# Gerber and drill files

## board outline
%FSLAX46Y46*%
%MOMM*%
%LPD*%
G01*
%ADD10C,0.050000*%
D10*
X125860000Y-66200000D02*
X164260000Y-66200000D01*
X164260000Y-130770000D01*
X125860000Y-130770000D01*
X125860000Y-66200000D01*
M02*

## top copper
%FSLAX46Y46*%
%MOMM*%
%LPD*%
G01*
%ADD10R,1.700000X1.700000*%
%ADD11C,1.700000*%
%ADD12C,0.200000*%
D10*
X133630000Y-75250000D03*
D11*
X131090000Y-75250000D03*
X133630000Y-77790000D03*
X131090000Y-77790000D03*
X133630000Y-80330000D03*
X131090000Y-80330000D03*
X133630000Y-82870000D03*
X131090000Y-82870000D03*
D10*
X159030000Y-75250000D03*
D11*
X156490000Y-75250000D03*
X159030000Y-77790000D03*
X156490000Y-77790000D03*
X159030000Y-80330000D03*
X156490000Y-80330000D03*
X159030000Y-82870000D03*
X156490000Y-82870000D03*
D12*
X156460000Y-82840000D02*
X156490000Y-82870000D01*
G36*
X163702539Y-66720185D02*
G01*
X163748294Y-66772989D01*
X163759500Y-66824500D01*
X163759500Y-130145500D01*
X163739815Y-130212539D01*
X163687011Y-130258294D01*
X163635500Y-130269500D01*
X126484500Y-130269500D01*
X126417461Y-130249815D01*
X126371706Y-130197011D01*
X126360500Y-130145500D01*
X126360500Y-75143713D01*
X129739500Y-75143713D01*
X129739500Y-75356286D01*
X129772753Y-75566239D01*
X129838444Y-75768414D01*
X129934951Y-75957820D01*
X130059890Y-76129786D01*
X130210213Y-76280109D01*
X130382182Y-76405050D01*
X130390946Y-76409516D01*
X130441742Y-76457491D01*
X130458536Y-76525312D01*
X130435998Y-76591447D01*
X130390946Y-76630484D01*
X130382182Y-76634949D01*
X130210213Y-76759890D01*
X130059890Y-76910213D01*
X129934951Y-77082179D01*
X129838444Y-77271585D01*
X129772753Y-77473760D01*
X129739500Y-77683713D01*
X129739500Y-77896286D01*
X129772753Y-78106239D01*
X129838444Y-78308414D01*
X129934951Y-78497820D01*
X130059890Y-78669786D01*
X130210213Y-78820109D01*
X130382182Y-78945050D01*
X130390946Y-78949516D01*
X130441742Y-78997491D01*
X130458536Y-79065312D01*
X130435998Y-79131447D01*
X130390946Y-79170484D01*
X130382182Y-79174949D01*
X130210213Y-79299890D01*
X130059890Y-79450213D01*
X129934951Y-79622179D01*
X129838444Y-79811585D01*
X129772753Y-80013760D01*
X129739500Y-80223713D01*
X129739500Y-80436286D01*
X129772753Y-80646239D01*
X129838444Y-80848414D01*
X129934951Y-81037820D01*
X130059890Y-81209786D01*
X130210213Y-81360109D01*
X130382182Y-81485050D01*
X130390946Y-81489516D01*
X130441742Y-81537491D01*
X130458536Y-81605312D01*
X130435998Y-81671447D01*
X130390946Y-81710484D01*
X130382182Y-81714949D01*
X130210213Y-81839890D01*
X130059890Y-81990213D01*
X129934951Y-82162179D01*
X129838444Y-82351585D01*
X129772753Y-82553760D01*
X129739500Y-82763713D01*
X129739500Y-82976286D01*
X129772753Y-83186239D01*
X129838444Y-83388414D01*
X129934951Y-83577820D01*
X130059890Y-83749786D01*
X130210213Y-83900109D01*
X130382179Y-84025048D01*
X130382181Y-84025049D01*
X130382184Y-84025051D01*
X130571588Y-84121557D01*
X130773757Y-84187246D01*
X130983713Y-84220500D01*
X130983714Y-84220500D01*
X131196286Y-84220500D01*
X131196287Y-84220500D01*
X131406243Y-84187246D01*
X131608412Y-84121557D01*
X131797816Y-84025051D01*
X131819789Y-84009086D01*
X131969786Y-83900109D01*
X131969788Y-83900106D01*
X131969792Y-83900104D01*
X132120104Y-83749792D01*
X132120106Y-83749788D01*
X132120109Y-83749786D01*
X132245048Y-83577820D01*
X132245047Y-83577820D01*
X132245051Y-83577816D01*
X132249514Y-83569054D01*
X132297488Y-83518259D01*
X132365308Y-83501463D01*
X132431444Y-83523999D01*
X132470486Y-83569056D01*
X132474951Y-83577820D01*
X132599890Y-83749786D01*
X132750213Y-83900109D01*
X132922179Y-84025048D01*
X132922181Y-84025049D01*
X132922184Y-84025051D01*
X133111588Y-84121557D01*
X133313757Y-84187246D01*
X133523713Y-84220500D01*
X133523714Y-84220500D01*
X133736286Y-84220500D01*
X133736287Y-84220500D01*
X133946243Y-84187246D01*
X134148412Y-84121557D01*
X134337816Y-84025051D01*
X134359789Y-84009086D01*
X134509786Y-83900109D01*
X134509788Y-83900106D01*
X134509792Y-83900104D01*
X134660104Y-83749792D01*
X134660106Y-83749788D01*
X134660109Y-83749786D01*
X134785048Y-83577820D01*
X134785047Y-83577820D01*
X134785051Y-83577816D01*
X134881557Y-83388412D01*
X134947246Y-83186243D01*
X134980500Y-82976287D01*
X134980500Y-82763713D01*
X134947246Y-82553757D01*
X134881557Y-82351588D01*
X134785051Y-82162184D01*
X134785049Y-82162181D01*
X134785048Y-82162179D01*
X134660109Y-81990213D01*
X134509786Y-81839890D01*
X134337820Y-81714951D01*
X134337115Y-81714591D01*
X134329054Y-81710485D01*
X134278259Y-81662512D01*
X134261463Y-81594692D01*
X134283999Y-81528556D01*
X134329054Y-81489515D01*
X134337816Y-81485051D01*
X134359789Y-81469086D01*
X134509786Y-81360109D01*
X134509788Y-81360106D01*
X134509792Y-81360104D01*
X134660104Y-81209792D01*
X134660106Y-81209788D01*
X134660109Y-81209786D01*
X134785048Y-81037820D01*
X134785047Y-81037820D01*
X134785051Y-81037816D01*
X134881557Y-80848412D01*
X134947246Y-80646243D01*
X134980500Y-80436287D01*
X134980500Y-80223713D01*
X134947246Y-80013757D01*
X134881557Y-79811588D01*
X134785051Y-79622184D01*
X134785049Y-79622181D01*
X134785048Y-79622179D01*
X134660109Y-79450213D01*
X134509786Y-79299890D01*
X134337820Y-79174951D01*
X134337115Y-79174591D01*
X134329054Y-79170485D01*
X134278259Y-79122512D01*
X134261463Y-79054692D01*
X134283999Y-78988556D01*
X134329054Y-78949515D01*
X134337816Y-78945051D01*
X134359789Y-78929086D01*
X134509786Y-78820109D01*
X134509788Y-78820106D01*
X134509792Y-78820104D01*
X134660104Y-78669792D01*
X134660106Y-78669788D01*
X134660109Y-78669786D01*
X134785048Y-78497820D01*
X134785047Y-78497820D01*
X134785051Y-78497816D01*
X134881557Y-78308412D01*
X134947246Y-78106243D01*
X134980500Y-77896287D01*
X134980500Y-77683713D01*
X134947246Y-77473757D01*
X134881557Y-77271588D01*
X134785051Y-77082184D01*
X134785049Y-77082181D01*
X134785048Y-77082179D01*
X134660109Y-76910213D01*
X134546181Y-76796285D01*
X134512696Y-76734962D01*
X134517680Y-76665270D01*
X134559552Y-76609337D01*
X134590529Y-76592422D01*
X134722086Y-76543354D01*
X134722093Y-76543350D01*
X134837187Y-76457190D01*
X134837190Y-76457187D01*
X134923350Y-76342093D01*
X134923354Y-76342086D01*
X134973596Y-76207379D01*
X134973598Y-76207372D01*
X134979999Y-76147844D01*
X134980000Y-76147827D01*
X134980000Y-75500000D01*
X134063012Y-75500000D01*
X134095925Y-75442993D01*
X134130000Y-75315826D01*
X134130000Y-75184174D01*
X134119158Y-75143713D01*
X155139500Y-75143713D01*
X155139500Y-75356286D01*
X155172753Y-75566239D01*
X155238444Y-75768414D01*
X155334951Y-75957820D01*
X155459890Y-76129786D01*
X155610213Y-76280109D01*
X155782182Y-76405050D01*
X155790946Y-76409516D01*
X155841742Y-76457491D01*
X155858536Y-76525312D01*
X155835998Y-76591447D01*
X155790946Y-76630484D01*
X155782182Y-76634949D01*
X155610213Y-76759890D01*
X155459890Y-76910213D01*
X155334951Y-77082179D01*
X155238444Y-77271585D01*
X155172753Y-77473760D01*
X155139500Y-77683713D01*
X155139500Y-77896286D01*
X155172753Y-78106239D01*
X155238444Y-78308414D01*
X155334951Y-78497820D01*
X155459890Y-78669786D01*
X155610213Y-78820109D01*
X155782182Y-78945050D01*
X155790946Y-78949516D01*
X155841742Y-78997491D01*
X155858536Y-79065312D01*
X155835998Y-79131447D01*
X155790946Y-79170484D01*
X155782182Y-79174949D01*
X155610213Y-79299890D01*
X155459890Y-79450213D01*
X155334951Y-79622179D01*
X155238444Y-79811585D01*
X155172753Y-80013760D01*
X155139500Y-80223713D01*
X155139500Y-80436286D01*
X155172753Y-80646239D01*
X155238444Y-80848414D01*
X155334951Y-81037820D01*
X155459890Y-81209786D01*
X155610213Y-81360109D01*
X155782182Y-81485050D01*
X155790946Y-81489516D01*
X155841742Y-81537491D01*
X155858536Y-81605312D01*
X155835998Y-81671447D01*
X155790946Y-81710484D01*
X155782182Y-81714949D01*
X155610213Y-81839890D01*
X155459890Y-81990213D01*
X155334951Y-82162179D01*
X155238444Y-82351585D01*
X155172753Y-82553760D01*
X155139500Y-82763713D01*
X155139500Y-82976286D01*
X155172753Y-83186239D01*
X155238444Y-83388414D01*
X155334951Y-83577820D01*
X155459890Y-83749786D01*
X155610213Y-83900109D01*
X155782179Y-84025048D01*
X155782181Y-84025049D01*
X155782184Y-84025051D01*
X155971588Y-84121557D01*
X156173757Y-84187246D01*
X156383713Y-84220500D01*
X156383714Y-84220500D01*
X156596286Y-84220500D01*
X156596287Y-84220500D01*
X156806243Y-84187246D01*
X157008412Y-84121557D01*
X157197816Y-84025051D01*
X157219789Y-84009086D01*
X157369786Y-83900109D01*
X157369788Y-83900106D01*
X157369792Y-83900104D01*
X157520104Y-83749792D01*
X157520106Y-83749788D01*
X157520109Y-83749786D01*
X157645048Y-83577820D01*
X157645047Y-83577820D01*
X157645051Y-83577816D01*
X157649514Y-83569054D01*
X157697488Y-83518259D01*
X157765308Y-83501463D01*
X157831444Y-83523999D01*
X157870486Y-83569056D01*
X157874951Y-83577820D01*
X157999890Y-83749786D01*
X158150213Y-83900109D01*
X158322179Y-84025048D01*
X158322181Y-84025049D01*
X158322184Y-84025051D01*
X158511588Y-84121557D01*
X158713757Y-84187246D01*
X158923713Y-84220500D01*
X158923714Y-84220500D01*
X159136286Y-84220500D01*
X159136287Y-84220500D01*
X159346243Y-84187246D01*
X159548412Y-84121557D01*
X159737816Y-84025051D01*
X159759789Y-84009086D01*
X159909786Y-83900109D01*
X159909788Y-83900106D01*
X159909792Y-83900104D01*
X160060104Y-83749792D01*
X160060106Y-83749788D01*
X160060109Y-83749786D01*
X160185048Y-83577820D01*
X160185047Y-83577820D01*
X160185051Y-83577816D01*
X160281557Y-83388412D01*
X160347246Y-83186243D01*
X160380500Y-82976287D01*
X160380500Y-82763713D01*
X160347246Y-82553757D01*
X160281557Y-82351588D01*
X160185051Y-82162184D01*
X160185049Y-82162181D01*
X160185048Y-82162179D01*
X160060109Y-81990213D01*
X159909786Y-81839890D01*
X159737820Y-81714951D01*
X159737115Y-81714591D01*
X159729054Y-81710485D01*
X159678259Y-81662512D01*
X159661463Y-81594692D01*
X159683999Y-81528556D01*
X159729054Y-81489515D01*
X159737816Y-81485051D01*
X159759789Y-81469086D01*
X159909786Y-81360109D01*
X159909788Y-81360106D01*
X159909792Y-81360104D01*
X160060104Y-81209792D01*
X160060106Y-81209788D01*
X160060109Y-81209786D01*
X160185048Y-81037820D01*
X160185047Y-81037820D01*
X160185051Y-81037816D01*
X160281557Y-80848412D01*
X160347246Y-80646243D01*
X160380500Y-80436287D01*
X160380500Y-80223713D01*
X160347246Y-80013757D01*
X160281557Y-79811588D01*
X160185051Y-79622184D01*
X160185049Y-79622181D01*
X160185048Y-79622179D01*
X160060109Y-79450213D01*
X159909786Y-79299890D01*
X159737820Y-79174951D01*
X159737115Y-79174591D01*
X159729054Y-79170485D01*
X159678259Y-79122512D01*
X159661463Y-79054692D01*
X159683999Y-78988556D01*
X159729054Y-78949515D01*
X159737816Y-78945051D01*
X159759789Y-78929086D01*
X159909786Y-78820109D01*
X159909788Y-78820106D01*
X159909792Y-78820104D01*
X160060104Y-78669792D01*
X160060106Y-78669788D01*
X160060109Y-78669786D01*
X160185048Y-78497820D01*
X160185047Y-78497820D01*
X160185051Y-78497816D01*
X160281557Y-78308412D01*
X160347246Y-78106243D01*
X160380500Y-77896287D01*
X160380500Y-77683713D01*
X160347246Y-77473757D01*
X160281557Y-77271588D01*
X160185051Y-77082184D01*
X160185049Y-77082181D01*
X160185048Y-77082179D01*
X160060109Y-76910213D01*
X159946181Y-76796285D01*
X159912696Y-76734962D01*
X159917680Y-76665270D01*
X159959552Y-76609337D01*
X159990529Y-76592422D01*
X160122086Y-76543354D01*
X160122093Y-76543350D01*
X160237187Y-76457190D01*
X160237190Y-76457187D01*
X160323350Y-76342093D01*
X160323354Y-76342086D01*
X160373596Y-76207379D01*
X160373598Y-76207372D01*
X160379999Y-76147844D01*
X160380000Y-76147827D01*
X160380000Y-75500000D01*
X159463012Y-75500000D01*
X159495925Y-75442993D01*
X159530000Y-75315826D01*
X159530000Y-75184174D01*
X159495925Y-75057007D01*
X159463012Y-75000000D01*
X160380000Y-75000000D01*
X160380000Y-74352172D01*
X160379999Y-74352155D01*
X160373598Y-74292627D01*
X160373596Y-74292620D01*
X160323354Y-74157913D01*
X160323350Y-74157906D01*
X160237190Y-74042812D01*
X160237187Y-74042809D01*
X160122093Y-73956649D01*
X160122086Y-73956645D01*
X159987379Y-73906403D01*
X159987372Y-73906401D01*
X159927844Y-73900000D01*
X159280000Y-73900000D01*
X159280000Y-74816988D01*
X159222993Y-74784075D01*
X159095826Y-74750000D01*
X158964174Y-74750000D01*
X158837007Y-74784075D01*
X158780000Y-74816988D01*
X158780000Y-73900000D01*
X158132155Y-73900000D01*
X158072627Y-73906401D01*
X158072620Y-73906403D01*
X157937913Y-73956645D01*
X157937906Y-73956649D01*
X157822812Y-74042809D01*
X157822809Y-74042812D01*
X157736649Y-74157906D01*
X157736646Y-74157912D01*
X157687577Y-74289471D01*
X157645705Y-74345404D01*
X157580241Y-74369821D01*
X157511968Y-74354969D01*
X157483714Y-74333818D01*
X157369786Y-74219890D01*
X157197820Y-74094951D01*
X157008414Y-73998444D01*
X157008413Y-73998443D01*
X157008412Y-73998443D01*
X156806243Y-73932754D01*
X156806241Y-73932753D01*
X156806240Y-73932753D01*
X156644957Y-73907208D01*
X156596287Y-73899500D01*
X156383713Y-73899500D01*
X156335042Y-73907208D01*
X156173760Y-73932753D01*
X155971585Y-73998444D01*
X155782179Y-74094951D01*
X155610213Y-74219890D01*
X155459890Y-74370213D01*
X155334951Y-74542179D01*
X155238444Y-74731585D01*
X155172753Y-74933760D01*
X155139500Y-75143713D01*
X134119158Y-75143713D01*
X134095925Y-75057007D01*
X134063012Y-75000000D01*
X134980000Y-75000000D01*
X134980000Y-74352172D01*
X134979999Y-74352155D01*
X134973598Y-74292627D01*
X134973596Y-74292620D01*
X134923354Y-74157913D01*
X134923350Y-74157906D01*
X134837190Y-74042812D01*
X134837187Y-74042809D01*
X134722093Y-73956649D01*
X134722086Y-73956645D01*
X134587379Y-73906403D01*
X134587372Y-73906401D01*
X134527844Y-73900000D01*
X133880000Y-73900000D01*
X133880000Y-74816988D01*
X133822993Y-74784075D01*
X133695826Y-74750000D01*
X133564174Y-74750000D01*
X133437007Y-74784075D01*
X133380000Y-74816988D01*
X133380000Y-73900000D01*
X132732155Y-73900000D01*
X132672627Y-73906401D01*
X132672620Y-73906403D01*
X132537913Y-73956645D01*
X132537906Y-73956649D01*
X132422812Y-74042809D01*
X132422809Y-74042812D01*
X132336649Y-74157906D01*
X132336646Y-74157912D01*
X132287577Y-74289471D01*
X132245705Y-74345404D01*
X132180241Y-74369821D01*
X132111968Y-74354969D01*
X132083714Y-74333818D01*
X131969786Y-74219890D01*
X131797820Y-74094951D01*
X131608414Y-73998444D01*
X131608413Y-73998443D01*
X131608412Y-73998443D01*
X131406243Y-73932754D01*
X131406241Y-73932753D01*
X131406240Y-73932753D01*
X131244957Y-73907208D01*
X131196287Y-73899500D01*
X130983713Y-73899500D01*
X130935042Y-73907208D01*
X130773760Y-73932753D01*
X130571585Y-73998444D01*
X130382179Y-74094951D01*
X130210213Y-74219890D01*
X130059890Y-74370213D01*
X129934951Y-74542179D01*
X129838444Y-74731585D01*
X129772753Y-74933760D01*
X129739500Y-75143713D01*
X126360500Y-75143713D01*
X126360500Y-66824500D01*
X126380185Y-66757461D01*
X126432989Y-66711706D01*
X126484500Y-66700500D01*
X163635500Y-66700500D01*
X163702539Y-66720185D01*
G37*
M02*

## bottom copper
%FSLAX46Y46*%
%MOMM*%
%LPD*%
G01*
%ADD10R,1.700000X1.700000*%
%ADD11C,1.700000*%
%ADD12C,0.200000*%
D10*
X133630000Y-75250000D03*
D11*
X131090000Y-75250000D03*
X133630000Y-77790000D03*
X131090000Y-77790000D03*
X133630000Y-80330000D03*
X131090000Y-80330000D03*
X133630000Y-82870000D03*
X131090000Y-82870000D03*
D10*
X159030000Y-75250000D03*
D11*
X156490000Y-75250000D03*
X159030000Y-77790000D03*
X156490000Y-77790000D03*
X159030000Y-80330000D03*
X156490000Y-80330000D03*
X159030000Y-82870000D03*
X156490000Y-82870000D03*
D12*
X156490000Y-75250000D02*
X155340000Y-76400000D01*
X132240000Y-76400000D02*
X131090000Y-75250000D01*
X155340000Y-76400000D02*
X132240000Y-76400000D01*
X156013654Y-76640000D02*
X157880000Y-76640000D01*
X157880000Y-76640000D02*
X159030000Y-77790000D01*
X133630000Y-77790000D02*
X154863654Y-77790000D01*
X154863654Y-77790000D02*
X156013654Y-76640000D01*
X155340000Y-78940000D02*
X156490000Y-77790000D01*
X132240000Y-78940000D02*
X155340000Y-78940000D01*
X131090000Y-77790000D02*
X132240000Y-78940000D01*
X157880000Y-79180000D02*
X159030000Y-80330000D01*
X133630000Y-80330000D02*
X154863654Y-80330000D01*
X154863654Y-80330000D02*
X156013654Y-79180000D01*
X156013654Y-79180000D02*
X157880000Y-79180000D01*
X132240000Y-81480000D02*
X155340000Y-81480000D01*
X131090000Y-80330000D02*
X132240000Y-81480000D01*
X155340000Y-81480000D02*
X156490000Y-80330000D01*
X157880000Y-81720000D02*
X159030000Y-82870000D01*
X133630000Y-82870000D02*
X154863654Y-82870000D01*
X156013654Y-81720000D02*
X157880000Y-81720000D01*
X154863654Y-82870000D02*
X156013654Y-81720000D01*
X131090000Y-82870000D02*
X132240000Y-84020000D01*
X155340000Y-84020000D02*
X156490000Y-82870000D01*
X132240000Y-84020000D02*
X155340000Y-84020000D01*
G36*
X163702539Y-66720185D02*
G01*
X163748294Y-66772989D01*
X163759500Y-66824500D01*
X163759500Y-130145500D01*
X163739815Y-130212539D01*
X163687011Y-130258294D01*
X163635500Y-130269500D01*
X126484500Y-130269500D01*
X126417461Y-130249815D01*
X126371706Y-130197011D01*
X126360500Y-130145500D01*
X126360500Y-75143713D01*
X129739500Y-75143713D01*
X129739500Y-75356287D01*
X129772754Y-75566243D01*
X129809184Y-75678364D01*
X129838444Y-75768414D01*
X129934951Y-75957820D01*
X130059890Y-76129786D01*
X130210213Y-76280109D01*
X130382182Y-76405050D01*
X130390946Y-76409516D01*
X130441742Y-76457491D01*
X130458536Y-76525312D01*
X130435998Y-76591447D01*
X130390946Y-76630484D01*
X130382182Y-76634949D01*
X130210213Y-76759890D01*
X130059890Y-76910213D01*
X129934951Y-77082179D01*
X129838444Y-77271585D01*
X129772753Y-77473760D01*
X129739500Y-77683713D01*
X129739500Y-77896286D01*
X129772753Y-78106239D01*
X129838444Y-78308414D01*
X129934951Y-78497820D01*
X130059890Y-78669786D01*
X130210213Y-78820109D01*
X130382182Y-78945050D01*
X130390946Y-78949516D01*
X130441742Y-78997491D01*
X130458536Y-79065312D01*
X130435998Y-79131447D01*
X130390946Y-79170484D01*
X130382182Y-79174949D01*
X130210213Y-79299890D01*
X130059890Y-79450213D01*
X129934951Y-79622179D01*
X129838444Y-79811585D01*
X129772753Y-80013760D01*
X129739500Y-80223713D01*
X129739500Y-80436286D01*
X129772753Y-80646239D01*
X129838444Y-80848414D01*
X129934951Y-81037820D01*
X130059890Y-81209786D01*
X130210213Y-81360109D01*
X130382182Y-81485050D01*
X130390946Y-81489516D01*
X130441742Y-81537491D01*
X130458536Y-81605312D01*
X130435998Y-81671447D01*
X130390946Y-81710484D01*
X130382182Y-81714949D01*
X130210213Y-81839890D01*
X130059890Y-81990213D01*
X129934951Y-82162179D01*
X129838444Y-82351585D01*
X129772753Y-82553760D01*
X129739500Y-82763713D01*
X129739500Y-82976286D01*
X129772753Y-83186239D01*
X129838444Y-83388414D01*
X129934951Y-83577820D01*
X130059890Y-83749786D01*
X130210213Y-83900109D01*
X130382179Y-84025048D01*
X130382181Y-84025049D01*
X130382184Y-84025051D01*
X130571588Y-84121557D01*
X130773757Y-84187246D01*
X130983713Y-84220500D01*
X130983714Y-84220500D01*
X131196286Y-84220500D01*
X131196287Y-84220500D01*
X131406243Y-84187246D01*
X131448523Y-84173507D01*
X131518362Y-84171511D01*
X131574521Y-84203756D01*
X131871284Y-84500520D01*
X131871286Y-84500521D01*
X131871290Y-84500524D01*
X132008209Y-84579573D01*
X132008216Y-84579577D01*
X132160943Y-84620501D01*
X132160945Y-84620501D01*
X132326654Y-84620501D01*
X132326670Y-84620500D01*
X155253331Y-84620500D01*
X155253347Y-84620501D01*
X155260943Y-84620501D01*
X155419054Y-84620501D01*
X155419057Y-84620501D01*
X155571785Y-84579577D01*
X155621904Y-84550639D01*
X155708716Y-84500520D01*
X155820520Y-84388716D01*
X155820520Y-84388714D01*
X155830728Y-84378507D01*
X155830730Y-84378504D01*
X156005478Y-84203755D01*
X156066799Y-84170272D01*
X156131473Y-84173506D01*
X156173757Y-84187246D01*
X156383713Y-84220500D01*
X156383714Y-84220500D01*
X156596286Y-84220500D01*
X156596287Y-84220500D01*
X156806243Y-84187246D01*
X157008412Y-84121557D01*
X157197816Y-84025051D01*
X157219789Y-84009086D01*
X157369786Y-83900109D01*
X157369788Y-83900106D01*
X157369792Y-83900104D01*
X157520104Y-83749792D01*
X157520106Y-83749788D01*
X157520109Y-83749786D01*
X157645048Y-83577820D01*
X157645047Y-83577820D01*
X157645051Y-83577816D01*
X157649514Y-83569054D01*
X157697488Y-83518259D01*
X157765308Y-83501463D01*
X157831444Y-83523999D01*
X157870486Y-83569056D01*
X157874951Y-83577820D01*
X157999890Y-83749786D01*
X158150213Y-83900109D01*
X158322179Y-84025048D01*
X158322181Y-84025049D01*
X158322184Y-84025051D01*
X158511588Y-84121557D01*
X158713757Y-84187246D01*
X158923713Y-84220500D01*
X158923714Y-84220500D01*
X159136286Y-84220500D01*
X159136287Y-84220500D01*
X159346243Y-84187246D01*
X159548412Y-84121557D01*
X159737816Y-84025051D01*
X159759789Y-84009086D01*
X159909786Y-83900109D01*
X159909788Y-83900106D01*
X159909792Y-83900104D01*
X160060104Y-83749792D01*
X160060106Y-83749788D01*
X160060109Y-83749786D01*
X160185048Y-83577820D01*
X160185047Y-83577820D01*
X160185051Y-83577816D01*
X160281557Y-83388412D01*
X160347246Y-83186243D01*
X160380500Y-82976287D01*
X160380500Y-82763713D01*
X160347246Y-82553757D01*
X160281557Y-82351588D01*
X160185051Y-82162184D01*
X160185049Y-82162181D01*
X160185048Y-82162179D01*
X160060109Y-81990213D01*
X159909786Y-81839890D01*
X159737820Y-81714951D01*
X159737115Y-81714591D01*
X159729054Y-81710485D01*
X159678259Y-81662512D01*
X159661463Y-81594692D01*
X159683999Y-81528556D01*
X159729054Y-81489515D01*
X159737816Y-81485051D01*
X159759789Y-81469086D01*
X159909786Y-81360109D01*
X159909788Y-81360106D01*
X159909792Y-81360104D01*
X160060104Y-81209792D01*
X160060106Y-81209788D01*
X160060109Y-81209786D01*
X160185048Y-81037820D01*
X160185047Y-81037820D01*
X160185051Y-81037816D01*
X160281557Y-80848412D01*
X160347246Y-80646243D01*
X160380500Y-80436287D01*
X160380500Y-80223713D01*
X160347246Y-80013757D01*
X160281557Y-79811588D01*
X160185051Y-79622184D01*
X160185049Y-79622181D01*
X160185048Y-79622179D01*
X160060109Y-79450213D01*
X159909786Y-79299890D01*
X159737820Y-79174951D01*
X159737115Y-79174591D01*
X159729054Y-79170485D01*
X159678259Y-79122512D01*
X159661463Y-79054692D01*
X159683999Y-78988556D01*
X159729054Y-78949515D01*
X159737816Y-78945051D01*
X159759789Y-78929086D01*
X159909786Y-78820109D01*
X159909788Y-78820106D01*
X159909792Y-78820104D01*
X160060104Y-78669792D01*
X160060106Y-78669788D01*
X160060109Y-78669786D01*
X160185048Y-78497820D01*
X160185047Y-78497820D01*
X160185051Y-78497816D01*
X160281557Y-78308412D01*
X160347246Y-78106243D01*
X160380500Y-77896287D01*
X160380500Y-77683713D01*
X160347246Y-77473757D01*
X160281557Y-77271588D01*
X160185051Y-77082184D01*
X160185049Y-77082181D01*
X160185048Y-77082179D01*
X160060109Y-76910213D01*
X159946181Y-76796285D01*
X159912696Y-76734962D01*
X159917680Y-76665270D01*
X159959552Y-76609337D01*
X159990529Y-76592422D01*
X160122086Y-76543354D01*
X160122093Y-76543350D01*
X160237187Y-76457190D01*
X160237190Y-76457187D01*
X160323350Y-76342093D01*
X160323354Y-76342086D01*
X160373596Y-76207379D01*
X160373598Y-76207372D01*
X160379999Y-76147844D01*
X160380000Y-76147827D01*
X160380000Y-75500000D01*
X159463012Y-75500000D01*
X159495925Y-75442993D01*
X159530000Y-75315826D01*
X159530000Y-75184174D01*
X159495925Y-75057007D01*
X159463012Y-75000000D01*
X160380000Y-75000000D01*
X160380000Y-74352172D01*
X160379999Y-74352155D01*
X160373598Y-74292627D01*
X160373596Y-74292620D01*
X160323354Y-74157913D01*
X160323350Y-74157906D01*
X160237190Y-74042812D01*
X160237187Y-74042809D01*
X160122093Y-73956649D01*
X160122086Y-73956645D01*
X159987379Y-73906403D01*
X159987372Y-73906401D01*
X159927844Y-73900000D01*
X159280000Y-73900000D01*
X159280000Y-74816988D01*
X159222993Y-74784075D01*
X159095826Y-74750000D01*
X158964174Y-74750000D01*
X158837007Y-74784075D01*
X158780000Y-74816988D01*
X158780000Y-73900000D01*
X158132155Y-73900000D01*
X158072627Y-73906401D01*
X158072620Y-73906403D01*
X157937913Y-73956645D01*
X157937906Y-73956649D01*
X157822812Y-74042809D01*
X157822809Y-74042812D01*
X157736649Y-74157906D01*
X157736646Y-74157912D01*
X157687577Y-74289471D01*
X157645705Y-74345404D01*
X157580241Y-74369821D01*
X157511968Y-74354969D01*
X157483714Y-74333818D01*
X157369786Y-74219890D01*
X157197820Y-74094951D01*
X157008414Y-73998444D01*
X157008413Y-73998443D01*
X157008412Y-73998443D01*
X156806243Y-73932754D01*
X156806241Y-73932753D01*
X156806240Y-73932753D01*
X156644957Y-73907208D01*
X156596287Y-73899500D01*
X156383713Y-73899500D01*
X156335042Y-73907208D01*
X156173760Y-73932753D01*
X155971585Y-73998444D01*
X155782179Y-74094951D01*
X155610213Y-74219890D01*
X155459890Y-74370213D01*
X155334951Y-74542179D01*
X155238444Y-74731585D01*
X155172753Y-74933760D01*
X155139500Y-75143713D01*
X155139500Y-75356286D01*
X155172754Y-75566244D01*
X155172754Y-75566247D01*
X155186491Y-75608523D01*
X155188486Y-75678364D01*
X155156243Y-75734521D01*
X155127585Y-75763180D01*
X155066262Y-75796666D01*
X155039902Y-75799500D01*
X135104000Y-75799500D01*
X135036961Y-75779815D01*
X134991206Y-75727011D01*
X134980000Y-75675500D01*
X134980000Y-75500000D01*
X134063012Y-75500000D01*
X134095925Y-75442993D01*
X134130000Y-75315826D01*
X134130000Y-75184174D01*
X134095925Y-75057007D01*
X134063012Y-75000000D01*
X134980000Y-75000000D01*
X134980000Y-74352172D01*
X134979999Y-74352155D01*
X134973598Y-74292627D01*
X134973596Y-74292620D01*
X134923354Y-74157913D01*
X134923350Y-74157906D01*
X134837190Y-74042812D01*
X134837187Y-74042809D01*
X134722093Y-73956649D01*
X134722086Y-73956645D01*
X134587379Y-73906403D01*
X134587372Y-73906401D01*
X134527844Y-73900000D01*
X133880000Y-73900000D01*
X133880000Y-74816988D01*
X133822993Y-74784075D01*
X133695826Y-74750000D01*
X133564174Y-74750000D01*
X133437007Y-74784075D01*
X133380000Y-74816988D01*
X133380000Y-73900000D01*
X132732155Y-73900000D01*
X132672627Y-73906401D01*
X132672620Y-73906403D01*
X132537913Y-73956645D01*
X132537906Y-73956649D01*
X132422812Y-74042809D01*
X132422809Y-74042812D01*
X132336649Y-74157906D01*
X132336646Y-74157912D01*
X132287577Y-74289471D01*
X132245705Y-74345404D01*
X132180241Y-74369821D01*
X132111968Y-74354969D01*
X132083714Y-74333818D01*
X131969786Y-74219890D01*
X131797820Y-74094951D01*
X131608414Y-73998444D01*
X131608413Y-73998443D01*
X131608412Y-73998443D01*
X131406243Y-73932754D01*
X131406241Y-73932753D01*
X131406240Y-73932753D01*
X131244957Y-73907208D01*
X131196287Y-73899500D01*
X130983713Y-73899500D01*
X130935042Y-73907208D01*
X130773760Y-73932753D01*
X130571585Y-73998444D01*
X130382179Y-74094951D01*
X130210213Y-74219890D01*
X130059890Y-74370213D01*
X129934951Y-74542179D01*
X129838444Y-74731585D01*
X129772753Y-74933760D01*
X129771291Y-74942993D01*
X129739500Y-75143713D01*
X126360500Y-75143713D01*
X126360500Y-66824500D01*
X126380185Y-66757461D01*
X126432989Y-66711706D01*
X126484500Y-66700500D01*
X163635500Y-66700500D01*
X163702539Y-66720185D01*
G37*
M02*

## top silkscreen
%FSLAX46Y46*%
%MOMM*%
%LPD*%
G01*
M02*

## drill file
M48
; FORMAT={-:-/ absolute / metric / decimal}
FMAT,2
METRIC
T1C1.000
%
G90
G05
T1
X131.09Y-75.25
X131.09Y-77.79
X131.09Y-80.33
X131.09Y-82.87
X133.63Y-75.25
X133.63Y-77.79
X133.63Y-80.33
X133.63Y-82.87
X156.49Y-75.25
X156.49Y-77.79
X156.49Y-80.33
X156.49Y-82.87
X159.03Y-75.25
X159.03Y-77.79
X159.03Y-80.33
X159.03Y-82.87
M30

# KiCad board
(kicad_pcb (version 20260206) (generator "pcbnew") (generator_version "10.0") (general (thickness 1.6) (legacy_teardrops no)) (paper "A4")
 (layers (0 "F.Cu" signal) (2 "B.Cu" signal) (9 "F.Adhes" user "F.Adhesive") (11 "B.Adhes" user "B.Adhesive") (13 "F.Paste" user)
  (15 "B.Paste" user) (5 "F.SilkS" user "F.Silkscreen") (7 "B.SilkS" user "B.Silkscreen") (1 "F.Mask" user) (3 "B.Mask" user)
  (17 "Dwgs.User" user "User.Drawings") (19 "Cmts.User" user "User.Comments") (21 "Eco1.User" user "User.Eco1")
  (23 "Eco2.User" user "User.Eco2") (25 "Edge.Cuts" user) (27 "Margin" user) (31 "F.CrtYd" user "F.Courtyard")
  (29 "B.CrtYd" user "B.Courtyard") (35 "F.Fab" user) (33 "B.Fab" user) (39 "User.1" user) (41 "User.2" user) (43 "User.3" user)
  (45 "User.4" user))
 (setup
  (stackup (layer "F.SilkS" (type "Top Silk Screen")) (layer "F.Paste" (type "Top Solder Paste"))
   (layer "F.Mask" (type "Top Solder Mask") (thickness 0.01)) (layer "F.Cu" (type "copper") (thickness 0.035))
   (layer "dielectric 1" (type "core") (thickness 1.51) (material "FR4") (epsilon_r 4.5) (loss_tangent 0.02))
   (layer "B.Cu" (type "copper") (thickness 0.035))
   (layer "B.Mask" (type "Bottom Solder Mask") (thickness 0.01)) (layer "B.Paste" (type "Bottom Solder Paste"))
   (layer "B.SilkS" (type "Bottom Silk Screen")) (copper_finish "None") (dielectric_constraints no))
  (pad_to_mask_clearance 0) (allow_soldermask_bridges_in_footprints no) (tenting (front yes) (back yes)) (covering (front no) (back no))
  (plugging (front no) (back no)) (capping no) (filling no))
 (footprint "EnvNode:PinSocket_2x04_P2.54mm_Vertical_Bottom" (layer "B.Cu") (at 131.09 75.25 180)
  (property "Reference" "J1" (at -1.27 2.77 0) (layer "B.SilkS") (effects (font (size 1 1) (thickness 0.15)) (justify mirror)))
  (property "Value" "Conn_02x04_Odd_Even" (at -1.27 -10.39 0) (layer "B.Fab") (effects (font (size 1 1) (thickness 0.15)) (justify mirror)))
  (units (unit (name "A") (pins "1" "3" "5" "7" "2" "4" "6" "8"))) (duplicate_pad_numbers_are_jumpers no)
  (pad "1" thru_hole rect (at -2.54 0 180) (size 1.7 1.7) (drill 1) (layers "*.Cu" "*.Mask") (remove_unused_layers no) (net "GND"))
  (pad "2" thru_hole circle (at 0 0 180) (size 1.7 1.7) (drill 1) (layers "*.Cu" "*.Mask") (remove_unused_layers no) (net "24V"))
  (pad "3" thru_hole circle (at -2.54 -2.54 180) (size 1.7 1.7) (drill 1) (layers "*.Cu" "*.Mask") (remove_unused_layers no) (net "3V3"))
  (pad "4" thru_hole circle (at 0 -2.54 180) (size 1.7 1.7) (drill 1) (layers "*.Cu" "*.Mask") (remove_unused_layers no) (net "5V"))
  (pad "5" thru_hole circle (at -2.54 -5.08 180) (size 1.7 1.7) (drill 1) (layers "*.Cu" "*.Mask") (remove_unused_layers no) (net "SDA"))
  (pad "6" thru_hole circle (at 0 -5.08 180) (size 1.7 1.7) (drill 1) (layers "*.Cu" "*.Mask") (remove_unused_layers no) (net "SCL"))
  (pad "7" thru_hole circle (at -2.54 -7.62 180) (size 1.7 1.7) (drill 1) (layers "*.Cu" "*.Mask") (remove_unused_layers no) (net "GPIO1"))
  (pad "8" thru_hole circle (at 0 -7.62 180) (size 1.7 1.7) (drill 1) (layers "*.Cu" "*.Mask") (remove_unused_layers no) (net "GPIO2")))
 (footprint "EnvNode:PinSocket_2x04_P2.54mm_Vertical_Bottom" (layer "B.Cu") (at 156.49 75.25 180)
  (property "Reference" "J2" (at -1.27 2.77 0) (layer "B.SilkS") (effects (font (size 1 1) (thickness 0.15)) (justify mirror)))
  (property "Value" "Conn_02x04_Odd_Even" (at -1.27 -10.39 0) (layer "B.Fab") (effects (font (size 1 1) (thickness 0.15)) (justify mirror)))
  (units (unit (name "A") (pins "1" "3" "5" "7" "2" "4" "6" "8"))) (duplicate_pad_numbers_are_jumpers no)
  (pad "1" thru_hole rect (at -2.54 0 180) (size 1.7 1.7) (drill 1) (layers "*.Cu" "*.Mask") (remove_unused_layers no) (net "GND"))
  (pad "2" thru_hole circle (at 0 0 180) (size 1.7 1.7) (drill 1) (layers "*.Cu" "*.Mask") (remove_unused_layers no) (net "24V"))
  (pad "3" thru_hole circle (at -2.54 -2.54 180) (size 1.7 1.7) (drill 1) (layers "*.Cu" "*.Mask") (remove_unused_layers no) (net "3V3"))
  (pad "4" thru_hole circle (at 0 -2.54 180) (size 1.7 1.7) (drill 1) (layers "*.Cu" "*.Mask") (remove_unused_layers no) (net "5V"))
  (pad "5" thru_hole circle (at -2.54 -5.08 180) (size 1.7 1.7) (drill 1) (layers "*.Cu" "*.Mask") (remove_unused_layers no) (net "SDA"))
  (pad "6" thru_hole circle (at 0 -5.08 180) (size 1.7 1.7) (drill 1) (layers "*.Cu" "*.Mask") (remove_unused_layers no) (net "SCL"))
  (pad "7" thru_hole circle (at -2.54 -7.62 180) (size 1.7 1.7) (drill 1) (layers "*.Cu" "*.Mask") (remove_unused_layers no) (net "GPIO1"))
  (pad "8" thru_hole circle (at 0 -7.62 180) (size 1.7 1.7) (drill 1) (layers "*.Cu" "*.Mask") (remove_unused_layers no) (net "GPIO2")))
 (gr_rect (start 125.86 66.2) (end 164.26 130.77) (stroke (width 0.05) (type default)) (fill no) (locked yes) (layer "Edge.Cuts"))
 (segment (start 156.49 75.25) (end 155.34 76.4) (width 0.2) (layer "B.Cu") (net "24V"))
 (segment (start 132.24 76.4) (end 131.09 75.25) (width 0.2) (layer "B.Cu") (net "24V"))
 (segment (start 155.34 76.4) (end 132.24 76.4) (width 0.2) (layer "B.Cu") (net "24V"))
 (segment (start 156.013654 76.64) (end 157.88 76.64) (width 0.2) (layer "B.Cu") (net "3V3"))
 (segment (start 157.88 76.64) (end 159.03 77.79) (width 0.2) (layer "B.Cu") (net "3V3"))
 (segment (start 133.63 77.79) (end 154.863654 77.79) (width 0.2) (layer "B.Cu") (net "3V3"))
 (segment (start 154.863654 77.79) (end 156.013654 76.64) (width 0.2) (layer "B.Cu") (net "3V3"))
 (segment (start 155.34 78.94) (end 156.49 77.79) (width 0.2) (layer "B.Cu") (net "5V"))
 (segment (start 132.24 78.94) (end 155.34 78.94) (width 0.2) (layer "B.Cu") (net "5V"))
 (segment (start 131.09 77.79) (end 132.24 78.94) (width 0.2) (layer "B.Cu") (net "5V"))
 (segment (start 157.88 79.18) (end 159.03 80.33) (width 0.2) (layer "B.Cu") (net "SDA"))
 (segment (start 133.63 80.33) (end 154.863654 80.33) (width 0.2) (layer "B.Cu") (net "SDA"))
 (segment (start 154.863654 80.33) (end 156.013654 79.18) (width 0.2) (layer "B.Cu") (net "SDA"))
 (segment (start 156.013654 79.18) (end 157.88 79.18) (width 0.2) (layer "B.Cu") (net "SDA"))
 (segment (start 132.24 81.48) (end 155.34 81.48) (width 0.2) (layer "B.Cu") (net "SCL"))
 (segment (start 131.09 80.33) (end 132.24 81.48) (width 0.2) (layer "B.Cu") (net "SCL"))
 (segment (start 155.34 81.48) (end 156.49 80.33) (width 0.2) (layer "B.Cu") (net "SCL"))
 (segment (start 157.88 81.72) (end 159.03 82.87) (width 0.2) (layer "B.Cu") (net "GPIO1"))
 (segment (start 133.63 82.87) (end 154.863654 82.87) (width 0.2) (layer "B.Cu") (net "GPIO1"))
 (segment (start 156.013654 81.72) (end 157.88 81.72) (width 0.2) (layer "B.Cu") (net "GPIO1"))
 (segment (start 154.863654 82.87) (end 156.013654 81.72) (width 0.2) (layer "B.Cu") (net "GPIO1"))
 (segment (start 156.46 82.84) (end 156.49 82.87) (width 0.2) (layer "F.Cu") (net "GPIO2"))
 (segment (start 131.09 82.87) (end 132.24 84.02) (width 0.2) (layer "B.Cu") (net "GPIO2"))
 (segment (start 155.34 84.02) (end 156.49 82.87) (width 0.2) (layer "B.Cu") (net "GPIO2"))
 (segment (start 132.24 84.02) (end 155.34 84.02) (width 0.2) (layer "B.Cu") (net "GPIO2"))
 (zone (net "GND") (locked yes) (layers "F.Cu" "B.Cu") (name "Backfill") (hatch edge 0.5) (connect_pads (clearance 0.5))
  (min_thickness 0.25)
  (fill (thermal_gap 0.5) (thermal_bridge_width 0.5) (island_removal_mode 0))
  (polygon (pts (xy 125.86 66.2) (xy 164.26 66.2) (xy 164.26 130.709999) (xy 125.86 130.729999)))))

